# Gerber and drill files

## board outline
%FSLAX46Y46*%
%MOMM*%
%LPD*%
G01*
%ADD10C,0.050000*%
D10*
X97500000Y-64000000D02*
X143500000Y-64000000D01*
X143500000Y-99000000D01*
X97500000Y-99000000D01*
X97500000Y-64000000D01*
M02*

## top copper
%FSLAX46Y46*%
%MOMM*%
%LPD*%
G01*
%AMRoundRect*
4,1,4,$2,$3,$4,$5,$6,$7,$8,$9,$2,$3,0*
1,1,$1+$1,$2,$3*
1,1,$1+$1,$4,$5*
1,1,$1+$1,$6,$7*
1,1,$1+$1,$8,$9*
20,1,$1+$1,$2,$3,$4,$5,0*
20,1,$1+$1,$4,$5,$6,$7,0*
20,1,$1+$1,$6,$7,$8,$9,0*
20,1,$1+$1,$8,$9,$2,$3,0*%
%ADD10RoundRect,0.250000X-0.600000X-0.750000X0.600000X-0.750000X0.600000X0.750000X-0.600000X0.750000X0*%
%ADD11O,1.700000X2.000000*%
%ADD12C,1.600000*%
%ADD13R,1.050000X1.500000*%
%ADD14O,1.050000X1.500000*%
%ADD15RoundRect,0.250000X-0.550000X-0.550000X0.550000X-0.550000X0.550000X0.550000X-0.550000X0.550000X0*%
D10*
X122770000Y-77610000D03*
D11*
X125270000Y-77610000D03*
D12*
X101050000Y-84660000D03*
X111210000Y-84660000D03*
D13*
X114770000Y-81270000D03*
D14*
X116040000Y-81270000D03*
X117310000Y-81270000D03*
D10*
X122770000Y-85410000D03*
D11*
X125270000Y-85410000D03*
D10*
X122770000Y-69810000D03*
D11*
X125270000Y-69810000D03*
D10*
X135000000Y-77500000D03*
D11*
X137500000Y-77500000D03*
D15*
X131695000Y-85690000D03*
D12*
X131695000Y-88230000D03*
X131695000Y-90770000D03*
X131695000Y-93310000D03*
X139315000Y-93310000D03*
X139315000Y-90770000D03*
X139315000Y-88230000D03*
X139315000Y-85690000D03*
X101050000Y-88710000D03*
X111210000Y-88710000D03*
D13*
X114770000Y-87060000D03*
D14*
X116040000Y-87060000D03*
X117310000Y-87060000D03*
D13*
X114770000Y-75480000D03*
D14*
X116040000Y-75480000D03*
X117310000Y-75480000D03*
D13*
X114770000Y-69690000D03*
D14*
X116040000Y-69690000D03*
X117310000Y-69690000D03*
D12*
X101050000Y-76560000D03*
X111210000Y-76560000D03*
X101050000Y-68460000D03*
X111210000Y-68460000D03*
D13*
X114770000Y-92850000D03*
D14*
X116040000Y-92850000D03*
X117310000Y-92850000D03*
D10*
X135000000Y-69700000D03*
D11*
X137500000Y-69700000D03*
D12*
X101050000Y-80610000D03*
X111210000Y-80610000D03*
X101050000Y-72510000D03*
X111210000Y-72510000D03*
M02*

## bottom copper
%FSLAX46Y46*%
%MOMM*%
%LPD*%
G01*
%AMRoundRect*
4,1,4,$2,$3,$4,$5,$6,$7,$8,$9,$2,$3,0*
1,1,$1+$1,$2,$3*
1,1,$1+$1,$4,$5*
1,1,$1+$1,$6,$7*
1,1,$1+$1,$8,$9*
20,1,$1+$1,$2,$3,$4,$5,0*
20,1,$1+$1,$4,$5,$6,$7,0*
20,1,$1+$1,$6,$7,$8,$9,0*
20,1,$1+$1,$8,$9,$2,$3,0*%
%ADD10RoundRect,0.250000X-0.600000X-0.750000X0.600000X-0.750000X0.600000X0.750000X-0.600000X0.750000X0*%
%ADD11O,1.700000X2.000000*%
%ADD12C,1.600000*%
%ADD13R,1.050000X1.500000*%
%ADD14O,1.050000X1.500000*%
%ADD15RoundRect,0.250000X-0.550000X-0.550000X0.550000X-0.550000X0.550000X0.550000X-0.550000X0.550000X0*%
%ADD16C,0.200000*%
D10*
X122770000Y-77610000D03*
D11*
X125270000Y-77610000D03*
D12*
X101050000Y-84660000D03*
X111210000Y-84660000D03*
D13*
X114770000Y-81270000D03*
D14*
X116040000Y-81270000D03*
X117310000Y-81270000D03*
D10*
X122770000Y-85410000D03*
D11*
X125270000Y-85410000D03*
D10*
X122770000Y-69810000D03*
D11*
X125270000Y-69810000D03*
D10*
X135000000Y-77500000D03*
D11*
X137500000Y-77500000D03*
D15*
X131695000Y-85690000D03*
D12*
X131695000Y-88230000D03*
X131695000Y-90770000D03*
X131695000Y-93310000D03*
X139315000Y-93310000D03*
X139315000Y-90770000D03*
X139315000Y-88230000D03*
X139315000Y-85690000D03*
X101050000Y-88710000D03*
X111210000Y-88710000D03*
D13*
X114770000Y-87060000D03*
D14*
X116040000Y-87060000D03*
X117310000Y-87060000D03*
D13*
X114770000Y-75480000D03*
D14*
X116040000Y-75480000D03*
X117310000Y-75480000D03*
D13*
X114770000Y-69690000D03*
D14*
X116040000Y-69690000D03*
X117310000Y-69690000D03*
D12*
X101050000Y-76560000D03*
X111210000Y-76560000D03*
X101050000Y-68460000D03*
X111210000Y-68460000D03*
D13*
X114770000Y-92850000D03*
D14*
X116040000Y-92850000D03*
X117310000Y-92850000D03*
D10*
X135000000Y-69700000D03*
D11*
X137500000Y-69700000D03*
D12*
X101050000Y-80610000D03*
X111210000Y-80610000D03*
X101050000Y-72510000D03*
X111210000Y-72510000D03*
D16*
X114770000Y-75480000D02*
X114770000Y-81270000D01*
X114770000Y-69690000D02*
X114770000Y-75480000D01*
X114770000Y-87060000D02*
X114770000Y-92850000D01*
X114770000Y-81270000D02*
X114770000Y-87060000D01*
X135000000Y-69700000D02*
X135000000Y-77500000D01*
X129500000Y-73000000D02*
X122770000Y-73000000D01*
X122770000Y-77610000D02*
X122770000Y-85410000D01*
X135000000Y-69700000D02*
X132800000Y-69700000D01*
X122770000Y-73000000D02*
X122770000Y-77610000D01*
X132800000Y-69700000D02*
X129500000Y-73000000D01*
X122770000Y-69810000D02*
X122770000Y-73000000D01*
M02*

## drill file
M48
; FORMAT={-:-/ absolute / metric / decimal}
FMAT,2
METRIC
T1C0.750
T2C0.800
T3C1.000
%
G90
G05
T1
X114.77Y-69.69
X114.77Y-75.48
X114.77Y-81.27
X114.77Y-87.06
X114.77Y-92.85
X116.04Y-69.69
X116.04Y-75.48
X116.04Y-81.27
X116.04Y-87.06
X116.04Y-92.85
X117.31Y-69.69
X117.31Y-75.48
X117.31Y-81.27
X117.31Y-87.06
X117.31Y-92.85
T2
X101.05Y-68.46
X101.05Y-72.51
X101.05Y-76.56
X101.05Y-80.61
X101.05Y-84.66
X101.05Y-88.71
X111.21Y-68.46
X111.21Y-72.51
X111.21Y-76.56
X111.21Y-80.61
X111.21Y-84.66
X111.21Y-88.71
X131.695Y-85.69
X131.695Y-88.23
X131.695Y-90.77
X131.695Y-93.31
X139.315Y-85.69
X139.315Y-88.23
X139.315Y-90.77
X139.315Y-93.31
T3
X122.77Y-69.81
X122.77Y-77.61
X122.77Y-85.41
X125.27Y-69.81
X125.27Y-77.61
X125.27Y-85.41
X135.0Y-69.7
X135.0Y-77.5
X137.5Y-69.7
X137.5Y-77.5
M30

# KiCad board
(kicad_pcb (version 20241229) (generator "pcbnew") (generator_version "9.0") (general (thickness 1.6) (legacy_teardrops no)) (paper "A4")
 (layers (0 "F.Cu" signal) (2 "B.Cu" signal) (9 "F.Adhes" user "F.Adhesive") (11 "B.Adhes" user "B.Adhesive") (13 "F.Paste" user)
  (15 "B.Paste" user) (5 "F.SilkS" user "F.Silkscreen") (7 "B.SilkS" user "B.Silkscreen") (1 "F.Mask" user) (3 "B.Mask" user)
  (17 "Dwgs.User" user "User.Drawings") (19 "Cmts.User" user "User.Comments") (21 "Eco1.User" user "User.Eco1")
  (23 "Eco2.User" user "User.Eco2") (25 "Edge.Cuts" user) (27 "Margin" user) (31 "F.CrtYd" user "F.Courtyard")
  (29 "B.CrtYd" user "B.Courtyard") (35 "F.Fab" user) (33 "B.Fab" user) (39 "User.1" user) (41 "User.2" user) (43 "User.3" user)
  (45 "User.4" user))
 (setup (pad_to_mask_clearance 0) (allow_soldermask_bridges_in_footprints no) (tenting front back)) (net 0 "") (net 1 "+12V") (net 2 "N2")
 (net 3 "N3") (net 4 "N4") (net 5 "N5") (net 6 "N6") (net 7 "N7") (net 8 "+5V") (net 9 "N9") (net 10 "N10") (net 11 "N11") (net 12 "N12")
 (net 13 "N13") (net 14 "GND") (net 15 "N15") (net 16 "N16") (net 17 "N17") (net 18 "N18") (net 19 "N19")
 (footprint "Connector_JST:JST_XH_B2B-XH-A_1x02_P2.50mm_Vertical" (layer "F.Cu") (at 122.77 77.61)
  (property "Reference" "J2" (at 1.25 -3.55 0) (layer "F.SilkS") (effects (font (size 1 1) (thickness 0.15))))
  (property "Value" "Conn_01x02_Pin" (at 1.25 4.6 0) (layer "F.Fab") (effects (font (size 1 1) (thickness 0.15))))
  (pad "1" thru_hole roundrect (at 0 0) (size 1.7 2) (drill 1) (layers "*.Cu" "*.Mask") (remove_unused_layers no)
   (roundrect_rratio 0.147059) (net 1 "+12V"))
  (pad "2" thru_hole oval (at 2.5 0) (size 1.7 2) (drill 1) (layers "*.Cu" "*.Mask") (remove_unused_layers no) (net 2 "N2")))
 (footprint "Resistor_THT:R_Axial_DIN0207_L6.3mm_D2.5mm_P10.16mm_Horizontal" (layer "F.Cu") (at 101.05 84.66)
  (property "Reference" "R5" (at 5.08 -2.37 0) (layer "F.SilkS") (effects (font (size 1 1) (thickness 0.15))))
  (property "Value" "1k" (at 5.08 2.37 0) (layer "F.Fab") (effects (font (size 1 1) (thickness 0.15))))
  (pad "1" thru_hole circle (at 0 0) (size 1.6 1.6) (drill 0.8) (layers "*.Cu" "*.Mask") (remove_unused_layers no) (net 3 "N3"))
  (pad "2" thru_hole circle (at 10.16 0) (size 1.6 1.6) (drill 0.8) (layers "*.Cu" "*.Mask") (remove_unused_layers no) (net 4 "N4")))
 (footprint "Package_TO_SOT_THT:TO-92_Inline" (layer "F.Cu") (at 114.77 81.27)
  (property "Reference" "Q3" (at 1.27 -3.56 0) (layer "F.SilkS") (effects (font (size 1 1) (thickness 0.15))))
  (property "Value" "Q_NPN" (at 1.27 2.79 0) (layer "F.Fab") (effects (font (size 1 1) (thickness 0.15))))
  (pad "1" thru_hole rect (at 0 0) (size 1.05 1.5) (drill 0.75) (layers "*.Cu" "*.Mask") (remove_unused_layers no))
  (pad "2" thru_hole oval (at 1.27 0) (size 1.05 1.5) (drill 0.75) (layers "*.Cu" "*.Mask") (remove_unused_layers no))
  (pad "3" thru_hole oval (at 2.54 0) (size 1.05 1.5) (drill 0.75) (layers "*.Cu" "*.Mask") (remove_unused_layers no)))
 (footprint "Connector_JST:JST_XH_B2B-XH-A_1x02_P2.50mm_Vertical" (layer "F.Cu") (at 122.77 85.41)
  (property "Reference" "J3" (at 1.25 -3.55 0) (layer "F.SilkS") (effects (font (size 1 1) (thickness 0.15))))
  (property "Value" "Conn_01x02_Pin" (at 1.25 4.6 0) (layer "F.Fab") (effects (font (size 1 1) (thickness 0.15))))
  (pad "1" thru_hole roundrect (at 0 0) (size 1.7 2) (drill 1) (layers "*.Cu" "*.Mask") (remove_unused_layers no)
   (roundrect_rratio 0.147059) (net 1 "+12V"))
  (pad "2" thru_hole oval (at 2.5 0) (size 1.7 2) (drill 1) (layers "*.Cu" "*.Mask") (remove_unused_layers no) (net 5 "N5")))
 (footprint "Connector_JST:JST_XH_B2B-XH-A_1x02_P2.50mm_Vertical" (layer "F.Cu") (at 122.77 69.81)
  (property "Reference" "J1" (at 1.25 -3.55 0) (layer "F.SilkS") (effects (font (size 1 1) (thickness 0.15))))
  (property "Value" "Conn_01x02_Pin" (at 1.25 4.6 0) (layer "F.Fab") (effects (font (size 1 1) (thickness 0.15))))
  (pad "1" thru_hole roundrect (at 0 0) (size 1.7 2) (drill 1) (layers "*.Cu" "*.Mask") (remove_unused_layers no)
   (roundrect_rratio 0.147059) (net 1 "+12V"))
  (pad "2" thru_hole oval (at 2.5 0) (size 1.7 2) (drill 1) (layers "*.Cu" "*.Mask") (remove_unused_layers no) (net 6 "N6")))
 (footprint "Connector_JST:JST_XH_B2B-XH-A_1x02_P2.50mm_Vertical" (layer "F.Cu") (at 135 77.5)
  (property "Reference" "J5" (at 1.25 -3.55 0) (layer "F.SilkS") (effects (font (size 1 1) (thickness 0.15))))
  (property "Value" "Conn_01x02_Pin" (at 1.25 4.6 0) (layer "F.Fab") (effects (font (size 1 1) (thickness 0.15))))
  (pad "1" thru_hole roundrect (at 0 0) (size 1.7 2) (drill 1) (layers "*.Cu" "*.Mask") (remove_unused_layers no)
   (roundrect_rratio 0.147059) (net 1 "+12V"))
  (pad "2" thru_hole oval (at 2.5 0) (size 1.7 2) (drill 1) (layers "*.Cu" "*.Mask") (remove_unused_layers no) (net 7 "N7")))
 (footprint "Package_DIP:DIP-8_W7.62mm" (layer "F.Cu") (at 131.695 85.69)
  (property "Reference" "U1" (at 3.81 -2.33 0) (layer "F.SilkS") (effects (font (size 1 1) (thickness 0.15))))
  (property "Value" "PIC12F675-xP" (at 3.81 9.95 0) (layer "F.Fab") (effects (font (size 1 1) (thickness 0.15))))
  (pad "1" thru_hole roundrect (at 0 0) (size 1.6 1.6) (drill 0.8) (layers "*.Cu" "*.Mask") (remove_unused_layers no)
   (roundrect_rratio 0.15625) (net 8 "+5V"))
  (pad "2" thru_hole circle (at 0 2.54) (size 1.6 1.6) (drill 0.8) (layers "*.Cu" "*.Mask") (remove_unused_layers no) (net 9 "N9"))
  (pad "3" thru_hole circle (at 0 5.08) (size 1.6 1.6) (drill 0.8) (layers "*.Cu" "*.Mask") (remove_unused_layers no) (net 3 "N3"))
  (pad "4" thru_hole circle (at 0 7.62) (size 1.6 1.6) (drill 0.8) (layers "*.Cu" "*.Mask") (remove_unused_layers no) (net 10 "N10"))
  (pad "5" thru_hole circle (at 7.62 7.62) (size 1.6 1.6) (drill 0.8) (layers "*.Cu" "*.Mask") (remove_unused_layers no) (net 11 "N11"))
  (pad "6" thru_hole circle (at 7.62 5.08) (size 1.6 1.6) (drill 0.8) (layers "*.Cu" "*.Mask") (remove_unused_layers no) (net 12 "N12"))
  (pad "7" thru_hole circle (at 7.62 2.54) (size 1.6 1.6) (drill 0.8) (layers "*.Cu" "*.Mask") (remove_unused_layers no) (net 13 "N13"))
  (pad "8" thru_hole circle (at 7.62 0) (size 1.6 1.6) (drill 0.8) (layers "*.Cu" "*.Mask") (remove_unused_layers no) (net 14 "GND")))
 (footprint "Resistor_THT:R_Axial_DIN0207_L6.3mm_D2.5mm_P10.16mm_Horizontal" (layer "F.Cu") (at 101.05 88.71)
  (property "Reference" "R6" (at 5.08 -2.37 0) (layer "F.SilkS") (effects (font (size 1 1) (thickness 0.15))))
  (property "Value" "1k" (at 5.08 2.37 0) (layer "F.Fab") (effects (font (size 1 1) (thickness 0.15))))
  (pad "1" thru_hole circle (at 0 0) (size 1.6 1.6) (drill 0.8) (layers "*.Cu" "*.Mask") (remove_unused_layers no) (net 9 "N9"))
  (pad "2" thru_hole circle (at 10.16 0) (size 1.6 1.6) (drill 0.8) (layers "*.Cu" "*.Mask") (remove_unused_layers no) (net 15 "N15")))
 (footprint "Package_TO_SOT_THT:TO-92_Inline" (layer "F.Cu") (at 114.77 87.06)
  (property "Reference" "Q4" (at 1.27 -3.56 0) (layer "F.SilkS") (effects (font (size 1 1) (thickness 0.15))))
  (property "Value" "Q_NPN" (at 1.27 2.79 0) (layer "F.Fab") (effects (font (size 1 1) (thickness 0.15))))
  (pad "1" thru_hole rect (at 0 0) (size 1.05 1.5) (drill 0.75) (layers "*.Cu" "*.Mask") (remove_unused_layers no))
  (pad "2" thru_hole oval (at 1.27 0) (size 1.05 1.5) (drill 0.75) (layers "*.Cu" "*.Mask") (remove_unused_layers no))
  (pad "3" thru_hole oval (at 2.54 0) (size 1.05 1.5) (drill 0.75) (layers "*.Cu" "*.Mask") (remove_unused_layers no)))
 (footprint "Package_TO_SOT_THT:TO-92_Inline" (layer "F.Cu") (at 114.77 75.48)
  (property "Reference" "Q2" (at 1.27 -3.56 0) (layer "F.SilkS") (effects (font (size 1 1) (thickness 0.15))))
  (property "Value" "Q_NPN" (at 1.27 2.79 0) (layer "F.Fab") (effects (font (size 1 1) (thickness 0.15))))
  (pad "1" thru_hole rect (at 0 0) (size 1.05 1.5) (drill 0.75) (layers "*.Cu" "*.Mask") (remove_unused_layers no))
  (pad "2" thru_hole oval (at 1.27 0) (size 1.05 1.5) (drill 0.75) (layers "*.Cu" "*.Mask") (remove_unused_layers no))
  (pad "3" thru_hole oval (at 2.54 0) (size 1.05 1.5) (drill 0.75) (layers "*.Cu" "*.Mask") (remove_unused_layers no)))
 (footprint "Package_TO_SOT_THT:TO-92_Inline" (layer "F.Cu") (at 114.77 69.69)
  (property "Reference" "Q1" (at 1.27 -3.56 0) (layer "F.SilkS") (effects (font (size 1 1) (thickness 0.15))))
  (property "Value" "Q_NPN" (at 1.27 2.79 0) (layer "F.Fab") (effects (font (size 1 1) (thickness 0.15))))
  (pad "1" thru_hole rect (at 0 0) (size 1.05 1.5) (drill 0.75) (layers "*.Cu" "*.Mask") (remove_unused_layers no))
  (pad "2" thru_hole oval (at 1.27 0) (size 1.05 1.5) (drill 0.75) (layers "*.Cu" "*.Mask") (remove_unused_layers no))
  (pad "3" thru_hole oval (at 2.54 0) (size 1.05 1.5) (drill 0.75) (layers "*.Cu" "*.Mask") (remove_unused_layers no)))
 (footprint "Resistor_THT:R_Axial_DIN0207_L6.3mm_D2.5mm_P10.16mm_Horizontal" (layer "F.Cu") (at 101.05 76.56)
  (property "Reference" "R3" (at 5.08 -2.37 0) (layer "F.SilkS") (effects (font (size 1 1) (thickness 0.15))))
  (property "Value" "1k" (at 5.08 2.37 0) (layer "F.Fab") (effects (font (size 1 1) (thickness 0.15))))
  (pad "1" thru_hole circle (at 0 0) (size 1.6 1.6) (drill 0.8) (layers "*.Cu" "*.Mask") (remove_unused_layers no) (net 12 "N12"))
  (pad "2" thru_hole circle (at 10.16 0) (size 1.6 1.6) (drill 0.8) (layers "*.Cu" "*.Mask") (remove_unused_layers no) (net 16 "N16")))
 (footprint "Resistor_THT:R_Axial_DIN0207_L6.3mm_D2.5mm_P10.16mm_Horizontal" (layer "F.Cu") (at 101.05 68.46)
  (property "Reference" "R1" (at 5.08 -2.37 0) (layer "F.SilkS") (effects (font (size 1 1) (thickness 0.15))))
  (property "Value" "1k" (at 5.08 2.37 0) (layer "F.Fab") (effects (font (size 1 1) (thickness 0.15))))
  (pad "1" thru_hole circle (at 0 0) (size 1.6 1.6) (drill 0.8) (layers "*.Cu" "*.Mask") (remove_unused_layers no) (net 10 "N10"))
  (pad "2" thru_hole circle (at 10.16 0) (size 1.6 1.6) (drill 0.8) (layers "*.Cu" "*.Mask") (remove_unused_layers no) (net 8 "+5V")))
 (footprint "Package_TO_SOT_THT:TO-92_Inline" (layer "F.Cu") (at 114.77 92.85)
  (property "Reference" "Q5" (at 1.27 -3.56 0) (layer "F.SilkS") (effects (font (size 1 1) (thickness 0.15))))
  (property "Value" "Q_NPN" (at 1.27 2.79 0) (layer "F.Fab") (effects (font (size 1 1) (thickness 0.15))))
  (pad "1" thru_hole rect (at 0 0) (size 1.05 1.5) (drill 0.75) (layers "*.Cu" "*.Mask") (remove_unused_layers no))
  (pad "2" thru_hole oval (at 1.27 0) (size 1.05 1.5) (drill 0.75) (layers "*.Cu" "*.Mask") (remove_unused_layers no))
  (pad "3" thru_hole oval (at 2.54 0) (size 1.05 1.5) (drill 0.75) (layers "*.Cu" "*.Mask") (remove_unused_layers no)))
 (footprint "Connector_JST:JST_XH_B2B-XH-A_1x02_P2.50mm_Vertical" (layer "F.Cu") (at 135 69.7)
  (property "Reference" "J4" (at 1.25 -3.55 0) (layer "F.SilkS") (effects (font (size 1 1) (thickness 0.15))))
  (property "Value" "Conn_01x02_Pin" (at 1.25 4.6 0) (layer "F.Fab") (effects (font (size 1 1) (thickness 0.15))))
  (pad "1" thru_hole roundrect (at 0 0) (size 1.7 2) (drill 1) (layers "*.Cu" "*.Mask") (remove_unused_layers no)
   (roundrect_rratio 0.147059) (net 1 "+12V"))
  (pad "2" thru_hole oval (at 2.5 0) (size 1.7 2) (drill 1) (layers "*.Cu" "*.Mask") (remove_unused_layers no) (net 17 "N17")))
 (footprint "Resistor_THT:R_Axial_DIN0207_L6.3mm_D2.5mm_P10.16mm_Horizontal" (layer "F.Cu") (at 101.05 80.61)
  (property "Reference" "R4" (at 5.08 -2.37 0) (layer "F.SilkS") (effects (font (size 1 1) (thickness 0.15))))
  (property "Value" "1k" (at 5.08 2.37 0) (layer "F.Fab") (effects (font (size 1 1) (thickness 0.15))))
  (pad "1" thru_hole circle (at 0 0) (size 1.6 1.6) (drill 0.8) (layers "*.Cu" "*.Mask") (remove_unused_layers no) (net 11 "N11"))
  (pad "2" thru_hole circle (at 10.16 0) (size 1.6 1.6) (drill 0.8) (layers "*.Cu" "*.Mask") (remove_unused_layers no) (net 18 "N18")))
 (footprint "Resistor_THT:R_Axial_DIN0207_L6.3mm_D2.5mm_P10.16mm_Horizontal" (layer "F.Cu") (at 101.05 72.51)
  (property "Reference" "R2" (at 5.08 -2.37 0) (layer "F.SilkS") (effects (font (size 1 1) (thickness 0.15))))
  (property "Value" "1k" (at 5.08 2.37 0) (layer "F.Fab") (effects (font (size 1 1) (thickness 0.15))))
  (pad "1" thru_hole circle (at 0 0) (size 1.6 1.6) (drill 0.8) (layers "*.Cu" "*.Mask") (remove_unused_layers no) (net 13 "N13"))
  (pad "2" thru_hole circle (at 10.16 0) (size 1.6 1.6) (drill 0.8) (layers "*.Cu" "*.Mask") (remove_unused_layers no) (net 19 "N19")))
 (gr_rect (start 97.5 64) (end 143.5 99) (stroke (width 0.05) (type default)) (fill no) (layer "Edge.Cuts"))
 (segment (start 114.77 75.48) (end 114.77 81.27) (width 0.2) (layer "B.Cu") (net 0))
 (segment (start 114.77 69.69) (end 114.77 75.48) (width 0.2) (layer "B.Cu") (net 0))
 (segment (start 114.77 87.06) (end 114.77 92.85) (width 0.2) (layer "B.Cu") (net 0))
 (segment (start 114.77 81.27) (end 114.77 87.06) (width 0.2) (layer "B.Cu") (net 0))
 (segment (start 135 69.7) (end 135 77.5) (width 0.2) (layer "B.Cu") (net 1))
 (segment (start 129.5 73) (end 122.77 73) (width 0.2) (layer "B.Cu") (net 1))
 (segment (start 122.77 77.61) (end 122.77 85.41) (width 0.2) (layer "B.Cu") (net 1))
 (segment (start 135 69.7) (end 132.8 69.7) (width 0.2) (layer "B.Cu") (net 1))
 (segment (start 122.77 73) (end 122.77 77.61) (width 0.2) (layer "B.Cu") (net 1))
 (segment (start 132.8 69.7) (end 129.5 73) (width 0.2) (layer "B.Cu") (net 1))
 (segment (start 122.77 69.81) (end 122.77 73) (width 0.2) (layer "B.Cu") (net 1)))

